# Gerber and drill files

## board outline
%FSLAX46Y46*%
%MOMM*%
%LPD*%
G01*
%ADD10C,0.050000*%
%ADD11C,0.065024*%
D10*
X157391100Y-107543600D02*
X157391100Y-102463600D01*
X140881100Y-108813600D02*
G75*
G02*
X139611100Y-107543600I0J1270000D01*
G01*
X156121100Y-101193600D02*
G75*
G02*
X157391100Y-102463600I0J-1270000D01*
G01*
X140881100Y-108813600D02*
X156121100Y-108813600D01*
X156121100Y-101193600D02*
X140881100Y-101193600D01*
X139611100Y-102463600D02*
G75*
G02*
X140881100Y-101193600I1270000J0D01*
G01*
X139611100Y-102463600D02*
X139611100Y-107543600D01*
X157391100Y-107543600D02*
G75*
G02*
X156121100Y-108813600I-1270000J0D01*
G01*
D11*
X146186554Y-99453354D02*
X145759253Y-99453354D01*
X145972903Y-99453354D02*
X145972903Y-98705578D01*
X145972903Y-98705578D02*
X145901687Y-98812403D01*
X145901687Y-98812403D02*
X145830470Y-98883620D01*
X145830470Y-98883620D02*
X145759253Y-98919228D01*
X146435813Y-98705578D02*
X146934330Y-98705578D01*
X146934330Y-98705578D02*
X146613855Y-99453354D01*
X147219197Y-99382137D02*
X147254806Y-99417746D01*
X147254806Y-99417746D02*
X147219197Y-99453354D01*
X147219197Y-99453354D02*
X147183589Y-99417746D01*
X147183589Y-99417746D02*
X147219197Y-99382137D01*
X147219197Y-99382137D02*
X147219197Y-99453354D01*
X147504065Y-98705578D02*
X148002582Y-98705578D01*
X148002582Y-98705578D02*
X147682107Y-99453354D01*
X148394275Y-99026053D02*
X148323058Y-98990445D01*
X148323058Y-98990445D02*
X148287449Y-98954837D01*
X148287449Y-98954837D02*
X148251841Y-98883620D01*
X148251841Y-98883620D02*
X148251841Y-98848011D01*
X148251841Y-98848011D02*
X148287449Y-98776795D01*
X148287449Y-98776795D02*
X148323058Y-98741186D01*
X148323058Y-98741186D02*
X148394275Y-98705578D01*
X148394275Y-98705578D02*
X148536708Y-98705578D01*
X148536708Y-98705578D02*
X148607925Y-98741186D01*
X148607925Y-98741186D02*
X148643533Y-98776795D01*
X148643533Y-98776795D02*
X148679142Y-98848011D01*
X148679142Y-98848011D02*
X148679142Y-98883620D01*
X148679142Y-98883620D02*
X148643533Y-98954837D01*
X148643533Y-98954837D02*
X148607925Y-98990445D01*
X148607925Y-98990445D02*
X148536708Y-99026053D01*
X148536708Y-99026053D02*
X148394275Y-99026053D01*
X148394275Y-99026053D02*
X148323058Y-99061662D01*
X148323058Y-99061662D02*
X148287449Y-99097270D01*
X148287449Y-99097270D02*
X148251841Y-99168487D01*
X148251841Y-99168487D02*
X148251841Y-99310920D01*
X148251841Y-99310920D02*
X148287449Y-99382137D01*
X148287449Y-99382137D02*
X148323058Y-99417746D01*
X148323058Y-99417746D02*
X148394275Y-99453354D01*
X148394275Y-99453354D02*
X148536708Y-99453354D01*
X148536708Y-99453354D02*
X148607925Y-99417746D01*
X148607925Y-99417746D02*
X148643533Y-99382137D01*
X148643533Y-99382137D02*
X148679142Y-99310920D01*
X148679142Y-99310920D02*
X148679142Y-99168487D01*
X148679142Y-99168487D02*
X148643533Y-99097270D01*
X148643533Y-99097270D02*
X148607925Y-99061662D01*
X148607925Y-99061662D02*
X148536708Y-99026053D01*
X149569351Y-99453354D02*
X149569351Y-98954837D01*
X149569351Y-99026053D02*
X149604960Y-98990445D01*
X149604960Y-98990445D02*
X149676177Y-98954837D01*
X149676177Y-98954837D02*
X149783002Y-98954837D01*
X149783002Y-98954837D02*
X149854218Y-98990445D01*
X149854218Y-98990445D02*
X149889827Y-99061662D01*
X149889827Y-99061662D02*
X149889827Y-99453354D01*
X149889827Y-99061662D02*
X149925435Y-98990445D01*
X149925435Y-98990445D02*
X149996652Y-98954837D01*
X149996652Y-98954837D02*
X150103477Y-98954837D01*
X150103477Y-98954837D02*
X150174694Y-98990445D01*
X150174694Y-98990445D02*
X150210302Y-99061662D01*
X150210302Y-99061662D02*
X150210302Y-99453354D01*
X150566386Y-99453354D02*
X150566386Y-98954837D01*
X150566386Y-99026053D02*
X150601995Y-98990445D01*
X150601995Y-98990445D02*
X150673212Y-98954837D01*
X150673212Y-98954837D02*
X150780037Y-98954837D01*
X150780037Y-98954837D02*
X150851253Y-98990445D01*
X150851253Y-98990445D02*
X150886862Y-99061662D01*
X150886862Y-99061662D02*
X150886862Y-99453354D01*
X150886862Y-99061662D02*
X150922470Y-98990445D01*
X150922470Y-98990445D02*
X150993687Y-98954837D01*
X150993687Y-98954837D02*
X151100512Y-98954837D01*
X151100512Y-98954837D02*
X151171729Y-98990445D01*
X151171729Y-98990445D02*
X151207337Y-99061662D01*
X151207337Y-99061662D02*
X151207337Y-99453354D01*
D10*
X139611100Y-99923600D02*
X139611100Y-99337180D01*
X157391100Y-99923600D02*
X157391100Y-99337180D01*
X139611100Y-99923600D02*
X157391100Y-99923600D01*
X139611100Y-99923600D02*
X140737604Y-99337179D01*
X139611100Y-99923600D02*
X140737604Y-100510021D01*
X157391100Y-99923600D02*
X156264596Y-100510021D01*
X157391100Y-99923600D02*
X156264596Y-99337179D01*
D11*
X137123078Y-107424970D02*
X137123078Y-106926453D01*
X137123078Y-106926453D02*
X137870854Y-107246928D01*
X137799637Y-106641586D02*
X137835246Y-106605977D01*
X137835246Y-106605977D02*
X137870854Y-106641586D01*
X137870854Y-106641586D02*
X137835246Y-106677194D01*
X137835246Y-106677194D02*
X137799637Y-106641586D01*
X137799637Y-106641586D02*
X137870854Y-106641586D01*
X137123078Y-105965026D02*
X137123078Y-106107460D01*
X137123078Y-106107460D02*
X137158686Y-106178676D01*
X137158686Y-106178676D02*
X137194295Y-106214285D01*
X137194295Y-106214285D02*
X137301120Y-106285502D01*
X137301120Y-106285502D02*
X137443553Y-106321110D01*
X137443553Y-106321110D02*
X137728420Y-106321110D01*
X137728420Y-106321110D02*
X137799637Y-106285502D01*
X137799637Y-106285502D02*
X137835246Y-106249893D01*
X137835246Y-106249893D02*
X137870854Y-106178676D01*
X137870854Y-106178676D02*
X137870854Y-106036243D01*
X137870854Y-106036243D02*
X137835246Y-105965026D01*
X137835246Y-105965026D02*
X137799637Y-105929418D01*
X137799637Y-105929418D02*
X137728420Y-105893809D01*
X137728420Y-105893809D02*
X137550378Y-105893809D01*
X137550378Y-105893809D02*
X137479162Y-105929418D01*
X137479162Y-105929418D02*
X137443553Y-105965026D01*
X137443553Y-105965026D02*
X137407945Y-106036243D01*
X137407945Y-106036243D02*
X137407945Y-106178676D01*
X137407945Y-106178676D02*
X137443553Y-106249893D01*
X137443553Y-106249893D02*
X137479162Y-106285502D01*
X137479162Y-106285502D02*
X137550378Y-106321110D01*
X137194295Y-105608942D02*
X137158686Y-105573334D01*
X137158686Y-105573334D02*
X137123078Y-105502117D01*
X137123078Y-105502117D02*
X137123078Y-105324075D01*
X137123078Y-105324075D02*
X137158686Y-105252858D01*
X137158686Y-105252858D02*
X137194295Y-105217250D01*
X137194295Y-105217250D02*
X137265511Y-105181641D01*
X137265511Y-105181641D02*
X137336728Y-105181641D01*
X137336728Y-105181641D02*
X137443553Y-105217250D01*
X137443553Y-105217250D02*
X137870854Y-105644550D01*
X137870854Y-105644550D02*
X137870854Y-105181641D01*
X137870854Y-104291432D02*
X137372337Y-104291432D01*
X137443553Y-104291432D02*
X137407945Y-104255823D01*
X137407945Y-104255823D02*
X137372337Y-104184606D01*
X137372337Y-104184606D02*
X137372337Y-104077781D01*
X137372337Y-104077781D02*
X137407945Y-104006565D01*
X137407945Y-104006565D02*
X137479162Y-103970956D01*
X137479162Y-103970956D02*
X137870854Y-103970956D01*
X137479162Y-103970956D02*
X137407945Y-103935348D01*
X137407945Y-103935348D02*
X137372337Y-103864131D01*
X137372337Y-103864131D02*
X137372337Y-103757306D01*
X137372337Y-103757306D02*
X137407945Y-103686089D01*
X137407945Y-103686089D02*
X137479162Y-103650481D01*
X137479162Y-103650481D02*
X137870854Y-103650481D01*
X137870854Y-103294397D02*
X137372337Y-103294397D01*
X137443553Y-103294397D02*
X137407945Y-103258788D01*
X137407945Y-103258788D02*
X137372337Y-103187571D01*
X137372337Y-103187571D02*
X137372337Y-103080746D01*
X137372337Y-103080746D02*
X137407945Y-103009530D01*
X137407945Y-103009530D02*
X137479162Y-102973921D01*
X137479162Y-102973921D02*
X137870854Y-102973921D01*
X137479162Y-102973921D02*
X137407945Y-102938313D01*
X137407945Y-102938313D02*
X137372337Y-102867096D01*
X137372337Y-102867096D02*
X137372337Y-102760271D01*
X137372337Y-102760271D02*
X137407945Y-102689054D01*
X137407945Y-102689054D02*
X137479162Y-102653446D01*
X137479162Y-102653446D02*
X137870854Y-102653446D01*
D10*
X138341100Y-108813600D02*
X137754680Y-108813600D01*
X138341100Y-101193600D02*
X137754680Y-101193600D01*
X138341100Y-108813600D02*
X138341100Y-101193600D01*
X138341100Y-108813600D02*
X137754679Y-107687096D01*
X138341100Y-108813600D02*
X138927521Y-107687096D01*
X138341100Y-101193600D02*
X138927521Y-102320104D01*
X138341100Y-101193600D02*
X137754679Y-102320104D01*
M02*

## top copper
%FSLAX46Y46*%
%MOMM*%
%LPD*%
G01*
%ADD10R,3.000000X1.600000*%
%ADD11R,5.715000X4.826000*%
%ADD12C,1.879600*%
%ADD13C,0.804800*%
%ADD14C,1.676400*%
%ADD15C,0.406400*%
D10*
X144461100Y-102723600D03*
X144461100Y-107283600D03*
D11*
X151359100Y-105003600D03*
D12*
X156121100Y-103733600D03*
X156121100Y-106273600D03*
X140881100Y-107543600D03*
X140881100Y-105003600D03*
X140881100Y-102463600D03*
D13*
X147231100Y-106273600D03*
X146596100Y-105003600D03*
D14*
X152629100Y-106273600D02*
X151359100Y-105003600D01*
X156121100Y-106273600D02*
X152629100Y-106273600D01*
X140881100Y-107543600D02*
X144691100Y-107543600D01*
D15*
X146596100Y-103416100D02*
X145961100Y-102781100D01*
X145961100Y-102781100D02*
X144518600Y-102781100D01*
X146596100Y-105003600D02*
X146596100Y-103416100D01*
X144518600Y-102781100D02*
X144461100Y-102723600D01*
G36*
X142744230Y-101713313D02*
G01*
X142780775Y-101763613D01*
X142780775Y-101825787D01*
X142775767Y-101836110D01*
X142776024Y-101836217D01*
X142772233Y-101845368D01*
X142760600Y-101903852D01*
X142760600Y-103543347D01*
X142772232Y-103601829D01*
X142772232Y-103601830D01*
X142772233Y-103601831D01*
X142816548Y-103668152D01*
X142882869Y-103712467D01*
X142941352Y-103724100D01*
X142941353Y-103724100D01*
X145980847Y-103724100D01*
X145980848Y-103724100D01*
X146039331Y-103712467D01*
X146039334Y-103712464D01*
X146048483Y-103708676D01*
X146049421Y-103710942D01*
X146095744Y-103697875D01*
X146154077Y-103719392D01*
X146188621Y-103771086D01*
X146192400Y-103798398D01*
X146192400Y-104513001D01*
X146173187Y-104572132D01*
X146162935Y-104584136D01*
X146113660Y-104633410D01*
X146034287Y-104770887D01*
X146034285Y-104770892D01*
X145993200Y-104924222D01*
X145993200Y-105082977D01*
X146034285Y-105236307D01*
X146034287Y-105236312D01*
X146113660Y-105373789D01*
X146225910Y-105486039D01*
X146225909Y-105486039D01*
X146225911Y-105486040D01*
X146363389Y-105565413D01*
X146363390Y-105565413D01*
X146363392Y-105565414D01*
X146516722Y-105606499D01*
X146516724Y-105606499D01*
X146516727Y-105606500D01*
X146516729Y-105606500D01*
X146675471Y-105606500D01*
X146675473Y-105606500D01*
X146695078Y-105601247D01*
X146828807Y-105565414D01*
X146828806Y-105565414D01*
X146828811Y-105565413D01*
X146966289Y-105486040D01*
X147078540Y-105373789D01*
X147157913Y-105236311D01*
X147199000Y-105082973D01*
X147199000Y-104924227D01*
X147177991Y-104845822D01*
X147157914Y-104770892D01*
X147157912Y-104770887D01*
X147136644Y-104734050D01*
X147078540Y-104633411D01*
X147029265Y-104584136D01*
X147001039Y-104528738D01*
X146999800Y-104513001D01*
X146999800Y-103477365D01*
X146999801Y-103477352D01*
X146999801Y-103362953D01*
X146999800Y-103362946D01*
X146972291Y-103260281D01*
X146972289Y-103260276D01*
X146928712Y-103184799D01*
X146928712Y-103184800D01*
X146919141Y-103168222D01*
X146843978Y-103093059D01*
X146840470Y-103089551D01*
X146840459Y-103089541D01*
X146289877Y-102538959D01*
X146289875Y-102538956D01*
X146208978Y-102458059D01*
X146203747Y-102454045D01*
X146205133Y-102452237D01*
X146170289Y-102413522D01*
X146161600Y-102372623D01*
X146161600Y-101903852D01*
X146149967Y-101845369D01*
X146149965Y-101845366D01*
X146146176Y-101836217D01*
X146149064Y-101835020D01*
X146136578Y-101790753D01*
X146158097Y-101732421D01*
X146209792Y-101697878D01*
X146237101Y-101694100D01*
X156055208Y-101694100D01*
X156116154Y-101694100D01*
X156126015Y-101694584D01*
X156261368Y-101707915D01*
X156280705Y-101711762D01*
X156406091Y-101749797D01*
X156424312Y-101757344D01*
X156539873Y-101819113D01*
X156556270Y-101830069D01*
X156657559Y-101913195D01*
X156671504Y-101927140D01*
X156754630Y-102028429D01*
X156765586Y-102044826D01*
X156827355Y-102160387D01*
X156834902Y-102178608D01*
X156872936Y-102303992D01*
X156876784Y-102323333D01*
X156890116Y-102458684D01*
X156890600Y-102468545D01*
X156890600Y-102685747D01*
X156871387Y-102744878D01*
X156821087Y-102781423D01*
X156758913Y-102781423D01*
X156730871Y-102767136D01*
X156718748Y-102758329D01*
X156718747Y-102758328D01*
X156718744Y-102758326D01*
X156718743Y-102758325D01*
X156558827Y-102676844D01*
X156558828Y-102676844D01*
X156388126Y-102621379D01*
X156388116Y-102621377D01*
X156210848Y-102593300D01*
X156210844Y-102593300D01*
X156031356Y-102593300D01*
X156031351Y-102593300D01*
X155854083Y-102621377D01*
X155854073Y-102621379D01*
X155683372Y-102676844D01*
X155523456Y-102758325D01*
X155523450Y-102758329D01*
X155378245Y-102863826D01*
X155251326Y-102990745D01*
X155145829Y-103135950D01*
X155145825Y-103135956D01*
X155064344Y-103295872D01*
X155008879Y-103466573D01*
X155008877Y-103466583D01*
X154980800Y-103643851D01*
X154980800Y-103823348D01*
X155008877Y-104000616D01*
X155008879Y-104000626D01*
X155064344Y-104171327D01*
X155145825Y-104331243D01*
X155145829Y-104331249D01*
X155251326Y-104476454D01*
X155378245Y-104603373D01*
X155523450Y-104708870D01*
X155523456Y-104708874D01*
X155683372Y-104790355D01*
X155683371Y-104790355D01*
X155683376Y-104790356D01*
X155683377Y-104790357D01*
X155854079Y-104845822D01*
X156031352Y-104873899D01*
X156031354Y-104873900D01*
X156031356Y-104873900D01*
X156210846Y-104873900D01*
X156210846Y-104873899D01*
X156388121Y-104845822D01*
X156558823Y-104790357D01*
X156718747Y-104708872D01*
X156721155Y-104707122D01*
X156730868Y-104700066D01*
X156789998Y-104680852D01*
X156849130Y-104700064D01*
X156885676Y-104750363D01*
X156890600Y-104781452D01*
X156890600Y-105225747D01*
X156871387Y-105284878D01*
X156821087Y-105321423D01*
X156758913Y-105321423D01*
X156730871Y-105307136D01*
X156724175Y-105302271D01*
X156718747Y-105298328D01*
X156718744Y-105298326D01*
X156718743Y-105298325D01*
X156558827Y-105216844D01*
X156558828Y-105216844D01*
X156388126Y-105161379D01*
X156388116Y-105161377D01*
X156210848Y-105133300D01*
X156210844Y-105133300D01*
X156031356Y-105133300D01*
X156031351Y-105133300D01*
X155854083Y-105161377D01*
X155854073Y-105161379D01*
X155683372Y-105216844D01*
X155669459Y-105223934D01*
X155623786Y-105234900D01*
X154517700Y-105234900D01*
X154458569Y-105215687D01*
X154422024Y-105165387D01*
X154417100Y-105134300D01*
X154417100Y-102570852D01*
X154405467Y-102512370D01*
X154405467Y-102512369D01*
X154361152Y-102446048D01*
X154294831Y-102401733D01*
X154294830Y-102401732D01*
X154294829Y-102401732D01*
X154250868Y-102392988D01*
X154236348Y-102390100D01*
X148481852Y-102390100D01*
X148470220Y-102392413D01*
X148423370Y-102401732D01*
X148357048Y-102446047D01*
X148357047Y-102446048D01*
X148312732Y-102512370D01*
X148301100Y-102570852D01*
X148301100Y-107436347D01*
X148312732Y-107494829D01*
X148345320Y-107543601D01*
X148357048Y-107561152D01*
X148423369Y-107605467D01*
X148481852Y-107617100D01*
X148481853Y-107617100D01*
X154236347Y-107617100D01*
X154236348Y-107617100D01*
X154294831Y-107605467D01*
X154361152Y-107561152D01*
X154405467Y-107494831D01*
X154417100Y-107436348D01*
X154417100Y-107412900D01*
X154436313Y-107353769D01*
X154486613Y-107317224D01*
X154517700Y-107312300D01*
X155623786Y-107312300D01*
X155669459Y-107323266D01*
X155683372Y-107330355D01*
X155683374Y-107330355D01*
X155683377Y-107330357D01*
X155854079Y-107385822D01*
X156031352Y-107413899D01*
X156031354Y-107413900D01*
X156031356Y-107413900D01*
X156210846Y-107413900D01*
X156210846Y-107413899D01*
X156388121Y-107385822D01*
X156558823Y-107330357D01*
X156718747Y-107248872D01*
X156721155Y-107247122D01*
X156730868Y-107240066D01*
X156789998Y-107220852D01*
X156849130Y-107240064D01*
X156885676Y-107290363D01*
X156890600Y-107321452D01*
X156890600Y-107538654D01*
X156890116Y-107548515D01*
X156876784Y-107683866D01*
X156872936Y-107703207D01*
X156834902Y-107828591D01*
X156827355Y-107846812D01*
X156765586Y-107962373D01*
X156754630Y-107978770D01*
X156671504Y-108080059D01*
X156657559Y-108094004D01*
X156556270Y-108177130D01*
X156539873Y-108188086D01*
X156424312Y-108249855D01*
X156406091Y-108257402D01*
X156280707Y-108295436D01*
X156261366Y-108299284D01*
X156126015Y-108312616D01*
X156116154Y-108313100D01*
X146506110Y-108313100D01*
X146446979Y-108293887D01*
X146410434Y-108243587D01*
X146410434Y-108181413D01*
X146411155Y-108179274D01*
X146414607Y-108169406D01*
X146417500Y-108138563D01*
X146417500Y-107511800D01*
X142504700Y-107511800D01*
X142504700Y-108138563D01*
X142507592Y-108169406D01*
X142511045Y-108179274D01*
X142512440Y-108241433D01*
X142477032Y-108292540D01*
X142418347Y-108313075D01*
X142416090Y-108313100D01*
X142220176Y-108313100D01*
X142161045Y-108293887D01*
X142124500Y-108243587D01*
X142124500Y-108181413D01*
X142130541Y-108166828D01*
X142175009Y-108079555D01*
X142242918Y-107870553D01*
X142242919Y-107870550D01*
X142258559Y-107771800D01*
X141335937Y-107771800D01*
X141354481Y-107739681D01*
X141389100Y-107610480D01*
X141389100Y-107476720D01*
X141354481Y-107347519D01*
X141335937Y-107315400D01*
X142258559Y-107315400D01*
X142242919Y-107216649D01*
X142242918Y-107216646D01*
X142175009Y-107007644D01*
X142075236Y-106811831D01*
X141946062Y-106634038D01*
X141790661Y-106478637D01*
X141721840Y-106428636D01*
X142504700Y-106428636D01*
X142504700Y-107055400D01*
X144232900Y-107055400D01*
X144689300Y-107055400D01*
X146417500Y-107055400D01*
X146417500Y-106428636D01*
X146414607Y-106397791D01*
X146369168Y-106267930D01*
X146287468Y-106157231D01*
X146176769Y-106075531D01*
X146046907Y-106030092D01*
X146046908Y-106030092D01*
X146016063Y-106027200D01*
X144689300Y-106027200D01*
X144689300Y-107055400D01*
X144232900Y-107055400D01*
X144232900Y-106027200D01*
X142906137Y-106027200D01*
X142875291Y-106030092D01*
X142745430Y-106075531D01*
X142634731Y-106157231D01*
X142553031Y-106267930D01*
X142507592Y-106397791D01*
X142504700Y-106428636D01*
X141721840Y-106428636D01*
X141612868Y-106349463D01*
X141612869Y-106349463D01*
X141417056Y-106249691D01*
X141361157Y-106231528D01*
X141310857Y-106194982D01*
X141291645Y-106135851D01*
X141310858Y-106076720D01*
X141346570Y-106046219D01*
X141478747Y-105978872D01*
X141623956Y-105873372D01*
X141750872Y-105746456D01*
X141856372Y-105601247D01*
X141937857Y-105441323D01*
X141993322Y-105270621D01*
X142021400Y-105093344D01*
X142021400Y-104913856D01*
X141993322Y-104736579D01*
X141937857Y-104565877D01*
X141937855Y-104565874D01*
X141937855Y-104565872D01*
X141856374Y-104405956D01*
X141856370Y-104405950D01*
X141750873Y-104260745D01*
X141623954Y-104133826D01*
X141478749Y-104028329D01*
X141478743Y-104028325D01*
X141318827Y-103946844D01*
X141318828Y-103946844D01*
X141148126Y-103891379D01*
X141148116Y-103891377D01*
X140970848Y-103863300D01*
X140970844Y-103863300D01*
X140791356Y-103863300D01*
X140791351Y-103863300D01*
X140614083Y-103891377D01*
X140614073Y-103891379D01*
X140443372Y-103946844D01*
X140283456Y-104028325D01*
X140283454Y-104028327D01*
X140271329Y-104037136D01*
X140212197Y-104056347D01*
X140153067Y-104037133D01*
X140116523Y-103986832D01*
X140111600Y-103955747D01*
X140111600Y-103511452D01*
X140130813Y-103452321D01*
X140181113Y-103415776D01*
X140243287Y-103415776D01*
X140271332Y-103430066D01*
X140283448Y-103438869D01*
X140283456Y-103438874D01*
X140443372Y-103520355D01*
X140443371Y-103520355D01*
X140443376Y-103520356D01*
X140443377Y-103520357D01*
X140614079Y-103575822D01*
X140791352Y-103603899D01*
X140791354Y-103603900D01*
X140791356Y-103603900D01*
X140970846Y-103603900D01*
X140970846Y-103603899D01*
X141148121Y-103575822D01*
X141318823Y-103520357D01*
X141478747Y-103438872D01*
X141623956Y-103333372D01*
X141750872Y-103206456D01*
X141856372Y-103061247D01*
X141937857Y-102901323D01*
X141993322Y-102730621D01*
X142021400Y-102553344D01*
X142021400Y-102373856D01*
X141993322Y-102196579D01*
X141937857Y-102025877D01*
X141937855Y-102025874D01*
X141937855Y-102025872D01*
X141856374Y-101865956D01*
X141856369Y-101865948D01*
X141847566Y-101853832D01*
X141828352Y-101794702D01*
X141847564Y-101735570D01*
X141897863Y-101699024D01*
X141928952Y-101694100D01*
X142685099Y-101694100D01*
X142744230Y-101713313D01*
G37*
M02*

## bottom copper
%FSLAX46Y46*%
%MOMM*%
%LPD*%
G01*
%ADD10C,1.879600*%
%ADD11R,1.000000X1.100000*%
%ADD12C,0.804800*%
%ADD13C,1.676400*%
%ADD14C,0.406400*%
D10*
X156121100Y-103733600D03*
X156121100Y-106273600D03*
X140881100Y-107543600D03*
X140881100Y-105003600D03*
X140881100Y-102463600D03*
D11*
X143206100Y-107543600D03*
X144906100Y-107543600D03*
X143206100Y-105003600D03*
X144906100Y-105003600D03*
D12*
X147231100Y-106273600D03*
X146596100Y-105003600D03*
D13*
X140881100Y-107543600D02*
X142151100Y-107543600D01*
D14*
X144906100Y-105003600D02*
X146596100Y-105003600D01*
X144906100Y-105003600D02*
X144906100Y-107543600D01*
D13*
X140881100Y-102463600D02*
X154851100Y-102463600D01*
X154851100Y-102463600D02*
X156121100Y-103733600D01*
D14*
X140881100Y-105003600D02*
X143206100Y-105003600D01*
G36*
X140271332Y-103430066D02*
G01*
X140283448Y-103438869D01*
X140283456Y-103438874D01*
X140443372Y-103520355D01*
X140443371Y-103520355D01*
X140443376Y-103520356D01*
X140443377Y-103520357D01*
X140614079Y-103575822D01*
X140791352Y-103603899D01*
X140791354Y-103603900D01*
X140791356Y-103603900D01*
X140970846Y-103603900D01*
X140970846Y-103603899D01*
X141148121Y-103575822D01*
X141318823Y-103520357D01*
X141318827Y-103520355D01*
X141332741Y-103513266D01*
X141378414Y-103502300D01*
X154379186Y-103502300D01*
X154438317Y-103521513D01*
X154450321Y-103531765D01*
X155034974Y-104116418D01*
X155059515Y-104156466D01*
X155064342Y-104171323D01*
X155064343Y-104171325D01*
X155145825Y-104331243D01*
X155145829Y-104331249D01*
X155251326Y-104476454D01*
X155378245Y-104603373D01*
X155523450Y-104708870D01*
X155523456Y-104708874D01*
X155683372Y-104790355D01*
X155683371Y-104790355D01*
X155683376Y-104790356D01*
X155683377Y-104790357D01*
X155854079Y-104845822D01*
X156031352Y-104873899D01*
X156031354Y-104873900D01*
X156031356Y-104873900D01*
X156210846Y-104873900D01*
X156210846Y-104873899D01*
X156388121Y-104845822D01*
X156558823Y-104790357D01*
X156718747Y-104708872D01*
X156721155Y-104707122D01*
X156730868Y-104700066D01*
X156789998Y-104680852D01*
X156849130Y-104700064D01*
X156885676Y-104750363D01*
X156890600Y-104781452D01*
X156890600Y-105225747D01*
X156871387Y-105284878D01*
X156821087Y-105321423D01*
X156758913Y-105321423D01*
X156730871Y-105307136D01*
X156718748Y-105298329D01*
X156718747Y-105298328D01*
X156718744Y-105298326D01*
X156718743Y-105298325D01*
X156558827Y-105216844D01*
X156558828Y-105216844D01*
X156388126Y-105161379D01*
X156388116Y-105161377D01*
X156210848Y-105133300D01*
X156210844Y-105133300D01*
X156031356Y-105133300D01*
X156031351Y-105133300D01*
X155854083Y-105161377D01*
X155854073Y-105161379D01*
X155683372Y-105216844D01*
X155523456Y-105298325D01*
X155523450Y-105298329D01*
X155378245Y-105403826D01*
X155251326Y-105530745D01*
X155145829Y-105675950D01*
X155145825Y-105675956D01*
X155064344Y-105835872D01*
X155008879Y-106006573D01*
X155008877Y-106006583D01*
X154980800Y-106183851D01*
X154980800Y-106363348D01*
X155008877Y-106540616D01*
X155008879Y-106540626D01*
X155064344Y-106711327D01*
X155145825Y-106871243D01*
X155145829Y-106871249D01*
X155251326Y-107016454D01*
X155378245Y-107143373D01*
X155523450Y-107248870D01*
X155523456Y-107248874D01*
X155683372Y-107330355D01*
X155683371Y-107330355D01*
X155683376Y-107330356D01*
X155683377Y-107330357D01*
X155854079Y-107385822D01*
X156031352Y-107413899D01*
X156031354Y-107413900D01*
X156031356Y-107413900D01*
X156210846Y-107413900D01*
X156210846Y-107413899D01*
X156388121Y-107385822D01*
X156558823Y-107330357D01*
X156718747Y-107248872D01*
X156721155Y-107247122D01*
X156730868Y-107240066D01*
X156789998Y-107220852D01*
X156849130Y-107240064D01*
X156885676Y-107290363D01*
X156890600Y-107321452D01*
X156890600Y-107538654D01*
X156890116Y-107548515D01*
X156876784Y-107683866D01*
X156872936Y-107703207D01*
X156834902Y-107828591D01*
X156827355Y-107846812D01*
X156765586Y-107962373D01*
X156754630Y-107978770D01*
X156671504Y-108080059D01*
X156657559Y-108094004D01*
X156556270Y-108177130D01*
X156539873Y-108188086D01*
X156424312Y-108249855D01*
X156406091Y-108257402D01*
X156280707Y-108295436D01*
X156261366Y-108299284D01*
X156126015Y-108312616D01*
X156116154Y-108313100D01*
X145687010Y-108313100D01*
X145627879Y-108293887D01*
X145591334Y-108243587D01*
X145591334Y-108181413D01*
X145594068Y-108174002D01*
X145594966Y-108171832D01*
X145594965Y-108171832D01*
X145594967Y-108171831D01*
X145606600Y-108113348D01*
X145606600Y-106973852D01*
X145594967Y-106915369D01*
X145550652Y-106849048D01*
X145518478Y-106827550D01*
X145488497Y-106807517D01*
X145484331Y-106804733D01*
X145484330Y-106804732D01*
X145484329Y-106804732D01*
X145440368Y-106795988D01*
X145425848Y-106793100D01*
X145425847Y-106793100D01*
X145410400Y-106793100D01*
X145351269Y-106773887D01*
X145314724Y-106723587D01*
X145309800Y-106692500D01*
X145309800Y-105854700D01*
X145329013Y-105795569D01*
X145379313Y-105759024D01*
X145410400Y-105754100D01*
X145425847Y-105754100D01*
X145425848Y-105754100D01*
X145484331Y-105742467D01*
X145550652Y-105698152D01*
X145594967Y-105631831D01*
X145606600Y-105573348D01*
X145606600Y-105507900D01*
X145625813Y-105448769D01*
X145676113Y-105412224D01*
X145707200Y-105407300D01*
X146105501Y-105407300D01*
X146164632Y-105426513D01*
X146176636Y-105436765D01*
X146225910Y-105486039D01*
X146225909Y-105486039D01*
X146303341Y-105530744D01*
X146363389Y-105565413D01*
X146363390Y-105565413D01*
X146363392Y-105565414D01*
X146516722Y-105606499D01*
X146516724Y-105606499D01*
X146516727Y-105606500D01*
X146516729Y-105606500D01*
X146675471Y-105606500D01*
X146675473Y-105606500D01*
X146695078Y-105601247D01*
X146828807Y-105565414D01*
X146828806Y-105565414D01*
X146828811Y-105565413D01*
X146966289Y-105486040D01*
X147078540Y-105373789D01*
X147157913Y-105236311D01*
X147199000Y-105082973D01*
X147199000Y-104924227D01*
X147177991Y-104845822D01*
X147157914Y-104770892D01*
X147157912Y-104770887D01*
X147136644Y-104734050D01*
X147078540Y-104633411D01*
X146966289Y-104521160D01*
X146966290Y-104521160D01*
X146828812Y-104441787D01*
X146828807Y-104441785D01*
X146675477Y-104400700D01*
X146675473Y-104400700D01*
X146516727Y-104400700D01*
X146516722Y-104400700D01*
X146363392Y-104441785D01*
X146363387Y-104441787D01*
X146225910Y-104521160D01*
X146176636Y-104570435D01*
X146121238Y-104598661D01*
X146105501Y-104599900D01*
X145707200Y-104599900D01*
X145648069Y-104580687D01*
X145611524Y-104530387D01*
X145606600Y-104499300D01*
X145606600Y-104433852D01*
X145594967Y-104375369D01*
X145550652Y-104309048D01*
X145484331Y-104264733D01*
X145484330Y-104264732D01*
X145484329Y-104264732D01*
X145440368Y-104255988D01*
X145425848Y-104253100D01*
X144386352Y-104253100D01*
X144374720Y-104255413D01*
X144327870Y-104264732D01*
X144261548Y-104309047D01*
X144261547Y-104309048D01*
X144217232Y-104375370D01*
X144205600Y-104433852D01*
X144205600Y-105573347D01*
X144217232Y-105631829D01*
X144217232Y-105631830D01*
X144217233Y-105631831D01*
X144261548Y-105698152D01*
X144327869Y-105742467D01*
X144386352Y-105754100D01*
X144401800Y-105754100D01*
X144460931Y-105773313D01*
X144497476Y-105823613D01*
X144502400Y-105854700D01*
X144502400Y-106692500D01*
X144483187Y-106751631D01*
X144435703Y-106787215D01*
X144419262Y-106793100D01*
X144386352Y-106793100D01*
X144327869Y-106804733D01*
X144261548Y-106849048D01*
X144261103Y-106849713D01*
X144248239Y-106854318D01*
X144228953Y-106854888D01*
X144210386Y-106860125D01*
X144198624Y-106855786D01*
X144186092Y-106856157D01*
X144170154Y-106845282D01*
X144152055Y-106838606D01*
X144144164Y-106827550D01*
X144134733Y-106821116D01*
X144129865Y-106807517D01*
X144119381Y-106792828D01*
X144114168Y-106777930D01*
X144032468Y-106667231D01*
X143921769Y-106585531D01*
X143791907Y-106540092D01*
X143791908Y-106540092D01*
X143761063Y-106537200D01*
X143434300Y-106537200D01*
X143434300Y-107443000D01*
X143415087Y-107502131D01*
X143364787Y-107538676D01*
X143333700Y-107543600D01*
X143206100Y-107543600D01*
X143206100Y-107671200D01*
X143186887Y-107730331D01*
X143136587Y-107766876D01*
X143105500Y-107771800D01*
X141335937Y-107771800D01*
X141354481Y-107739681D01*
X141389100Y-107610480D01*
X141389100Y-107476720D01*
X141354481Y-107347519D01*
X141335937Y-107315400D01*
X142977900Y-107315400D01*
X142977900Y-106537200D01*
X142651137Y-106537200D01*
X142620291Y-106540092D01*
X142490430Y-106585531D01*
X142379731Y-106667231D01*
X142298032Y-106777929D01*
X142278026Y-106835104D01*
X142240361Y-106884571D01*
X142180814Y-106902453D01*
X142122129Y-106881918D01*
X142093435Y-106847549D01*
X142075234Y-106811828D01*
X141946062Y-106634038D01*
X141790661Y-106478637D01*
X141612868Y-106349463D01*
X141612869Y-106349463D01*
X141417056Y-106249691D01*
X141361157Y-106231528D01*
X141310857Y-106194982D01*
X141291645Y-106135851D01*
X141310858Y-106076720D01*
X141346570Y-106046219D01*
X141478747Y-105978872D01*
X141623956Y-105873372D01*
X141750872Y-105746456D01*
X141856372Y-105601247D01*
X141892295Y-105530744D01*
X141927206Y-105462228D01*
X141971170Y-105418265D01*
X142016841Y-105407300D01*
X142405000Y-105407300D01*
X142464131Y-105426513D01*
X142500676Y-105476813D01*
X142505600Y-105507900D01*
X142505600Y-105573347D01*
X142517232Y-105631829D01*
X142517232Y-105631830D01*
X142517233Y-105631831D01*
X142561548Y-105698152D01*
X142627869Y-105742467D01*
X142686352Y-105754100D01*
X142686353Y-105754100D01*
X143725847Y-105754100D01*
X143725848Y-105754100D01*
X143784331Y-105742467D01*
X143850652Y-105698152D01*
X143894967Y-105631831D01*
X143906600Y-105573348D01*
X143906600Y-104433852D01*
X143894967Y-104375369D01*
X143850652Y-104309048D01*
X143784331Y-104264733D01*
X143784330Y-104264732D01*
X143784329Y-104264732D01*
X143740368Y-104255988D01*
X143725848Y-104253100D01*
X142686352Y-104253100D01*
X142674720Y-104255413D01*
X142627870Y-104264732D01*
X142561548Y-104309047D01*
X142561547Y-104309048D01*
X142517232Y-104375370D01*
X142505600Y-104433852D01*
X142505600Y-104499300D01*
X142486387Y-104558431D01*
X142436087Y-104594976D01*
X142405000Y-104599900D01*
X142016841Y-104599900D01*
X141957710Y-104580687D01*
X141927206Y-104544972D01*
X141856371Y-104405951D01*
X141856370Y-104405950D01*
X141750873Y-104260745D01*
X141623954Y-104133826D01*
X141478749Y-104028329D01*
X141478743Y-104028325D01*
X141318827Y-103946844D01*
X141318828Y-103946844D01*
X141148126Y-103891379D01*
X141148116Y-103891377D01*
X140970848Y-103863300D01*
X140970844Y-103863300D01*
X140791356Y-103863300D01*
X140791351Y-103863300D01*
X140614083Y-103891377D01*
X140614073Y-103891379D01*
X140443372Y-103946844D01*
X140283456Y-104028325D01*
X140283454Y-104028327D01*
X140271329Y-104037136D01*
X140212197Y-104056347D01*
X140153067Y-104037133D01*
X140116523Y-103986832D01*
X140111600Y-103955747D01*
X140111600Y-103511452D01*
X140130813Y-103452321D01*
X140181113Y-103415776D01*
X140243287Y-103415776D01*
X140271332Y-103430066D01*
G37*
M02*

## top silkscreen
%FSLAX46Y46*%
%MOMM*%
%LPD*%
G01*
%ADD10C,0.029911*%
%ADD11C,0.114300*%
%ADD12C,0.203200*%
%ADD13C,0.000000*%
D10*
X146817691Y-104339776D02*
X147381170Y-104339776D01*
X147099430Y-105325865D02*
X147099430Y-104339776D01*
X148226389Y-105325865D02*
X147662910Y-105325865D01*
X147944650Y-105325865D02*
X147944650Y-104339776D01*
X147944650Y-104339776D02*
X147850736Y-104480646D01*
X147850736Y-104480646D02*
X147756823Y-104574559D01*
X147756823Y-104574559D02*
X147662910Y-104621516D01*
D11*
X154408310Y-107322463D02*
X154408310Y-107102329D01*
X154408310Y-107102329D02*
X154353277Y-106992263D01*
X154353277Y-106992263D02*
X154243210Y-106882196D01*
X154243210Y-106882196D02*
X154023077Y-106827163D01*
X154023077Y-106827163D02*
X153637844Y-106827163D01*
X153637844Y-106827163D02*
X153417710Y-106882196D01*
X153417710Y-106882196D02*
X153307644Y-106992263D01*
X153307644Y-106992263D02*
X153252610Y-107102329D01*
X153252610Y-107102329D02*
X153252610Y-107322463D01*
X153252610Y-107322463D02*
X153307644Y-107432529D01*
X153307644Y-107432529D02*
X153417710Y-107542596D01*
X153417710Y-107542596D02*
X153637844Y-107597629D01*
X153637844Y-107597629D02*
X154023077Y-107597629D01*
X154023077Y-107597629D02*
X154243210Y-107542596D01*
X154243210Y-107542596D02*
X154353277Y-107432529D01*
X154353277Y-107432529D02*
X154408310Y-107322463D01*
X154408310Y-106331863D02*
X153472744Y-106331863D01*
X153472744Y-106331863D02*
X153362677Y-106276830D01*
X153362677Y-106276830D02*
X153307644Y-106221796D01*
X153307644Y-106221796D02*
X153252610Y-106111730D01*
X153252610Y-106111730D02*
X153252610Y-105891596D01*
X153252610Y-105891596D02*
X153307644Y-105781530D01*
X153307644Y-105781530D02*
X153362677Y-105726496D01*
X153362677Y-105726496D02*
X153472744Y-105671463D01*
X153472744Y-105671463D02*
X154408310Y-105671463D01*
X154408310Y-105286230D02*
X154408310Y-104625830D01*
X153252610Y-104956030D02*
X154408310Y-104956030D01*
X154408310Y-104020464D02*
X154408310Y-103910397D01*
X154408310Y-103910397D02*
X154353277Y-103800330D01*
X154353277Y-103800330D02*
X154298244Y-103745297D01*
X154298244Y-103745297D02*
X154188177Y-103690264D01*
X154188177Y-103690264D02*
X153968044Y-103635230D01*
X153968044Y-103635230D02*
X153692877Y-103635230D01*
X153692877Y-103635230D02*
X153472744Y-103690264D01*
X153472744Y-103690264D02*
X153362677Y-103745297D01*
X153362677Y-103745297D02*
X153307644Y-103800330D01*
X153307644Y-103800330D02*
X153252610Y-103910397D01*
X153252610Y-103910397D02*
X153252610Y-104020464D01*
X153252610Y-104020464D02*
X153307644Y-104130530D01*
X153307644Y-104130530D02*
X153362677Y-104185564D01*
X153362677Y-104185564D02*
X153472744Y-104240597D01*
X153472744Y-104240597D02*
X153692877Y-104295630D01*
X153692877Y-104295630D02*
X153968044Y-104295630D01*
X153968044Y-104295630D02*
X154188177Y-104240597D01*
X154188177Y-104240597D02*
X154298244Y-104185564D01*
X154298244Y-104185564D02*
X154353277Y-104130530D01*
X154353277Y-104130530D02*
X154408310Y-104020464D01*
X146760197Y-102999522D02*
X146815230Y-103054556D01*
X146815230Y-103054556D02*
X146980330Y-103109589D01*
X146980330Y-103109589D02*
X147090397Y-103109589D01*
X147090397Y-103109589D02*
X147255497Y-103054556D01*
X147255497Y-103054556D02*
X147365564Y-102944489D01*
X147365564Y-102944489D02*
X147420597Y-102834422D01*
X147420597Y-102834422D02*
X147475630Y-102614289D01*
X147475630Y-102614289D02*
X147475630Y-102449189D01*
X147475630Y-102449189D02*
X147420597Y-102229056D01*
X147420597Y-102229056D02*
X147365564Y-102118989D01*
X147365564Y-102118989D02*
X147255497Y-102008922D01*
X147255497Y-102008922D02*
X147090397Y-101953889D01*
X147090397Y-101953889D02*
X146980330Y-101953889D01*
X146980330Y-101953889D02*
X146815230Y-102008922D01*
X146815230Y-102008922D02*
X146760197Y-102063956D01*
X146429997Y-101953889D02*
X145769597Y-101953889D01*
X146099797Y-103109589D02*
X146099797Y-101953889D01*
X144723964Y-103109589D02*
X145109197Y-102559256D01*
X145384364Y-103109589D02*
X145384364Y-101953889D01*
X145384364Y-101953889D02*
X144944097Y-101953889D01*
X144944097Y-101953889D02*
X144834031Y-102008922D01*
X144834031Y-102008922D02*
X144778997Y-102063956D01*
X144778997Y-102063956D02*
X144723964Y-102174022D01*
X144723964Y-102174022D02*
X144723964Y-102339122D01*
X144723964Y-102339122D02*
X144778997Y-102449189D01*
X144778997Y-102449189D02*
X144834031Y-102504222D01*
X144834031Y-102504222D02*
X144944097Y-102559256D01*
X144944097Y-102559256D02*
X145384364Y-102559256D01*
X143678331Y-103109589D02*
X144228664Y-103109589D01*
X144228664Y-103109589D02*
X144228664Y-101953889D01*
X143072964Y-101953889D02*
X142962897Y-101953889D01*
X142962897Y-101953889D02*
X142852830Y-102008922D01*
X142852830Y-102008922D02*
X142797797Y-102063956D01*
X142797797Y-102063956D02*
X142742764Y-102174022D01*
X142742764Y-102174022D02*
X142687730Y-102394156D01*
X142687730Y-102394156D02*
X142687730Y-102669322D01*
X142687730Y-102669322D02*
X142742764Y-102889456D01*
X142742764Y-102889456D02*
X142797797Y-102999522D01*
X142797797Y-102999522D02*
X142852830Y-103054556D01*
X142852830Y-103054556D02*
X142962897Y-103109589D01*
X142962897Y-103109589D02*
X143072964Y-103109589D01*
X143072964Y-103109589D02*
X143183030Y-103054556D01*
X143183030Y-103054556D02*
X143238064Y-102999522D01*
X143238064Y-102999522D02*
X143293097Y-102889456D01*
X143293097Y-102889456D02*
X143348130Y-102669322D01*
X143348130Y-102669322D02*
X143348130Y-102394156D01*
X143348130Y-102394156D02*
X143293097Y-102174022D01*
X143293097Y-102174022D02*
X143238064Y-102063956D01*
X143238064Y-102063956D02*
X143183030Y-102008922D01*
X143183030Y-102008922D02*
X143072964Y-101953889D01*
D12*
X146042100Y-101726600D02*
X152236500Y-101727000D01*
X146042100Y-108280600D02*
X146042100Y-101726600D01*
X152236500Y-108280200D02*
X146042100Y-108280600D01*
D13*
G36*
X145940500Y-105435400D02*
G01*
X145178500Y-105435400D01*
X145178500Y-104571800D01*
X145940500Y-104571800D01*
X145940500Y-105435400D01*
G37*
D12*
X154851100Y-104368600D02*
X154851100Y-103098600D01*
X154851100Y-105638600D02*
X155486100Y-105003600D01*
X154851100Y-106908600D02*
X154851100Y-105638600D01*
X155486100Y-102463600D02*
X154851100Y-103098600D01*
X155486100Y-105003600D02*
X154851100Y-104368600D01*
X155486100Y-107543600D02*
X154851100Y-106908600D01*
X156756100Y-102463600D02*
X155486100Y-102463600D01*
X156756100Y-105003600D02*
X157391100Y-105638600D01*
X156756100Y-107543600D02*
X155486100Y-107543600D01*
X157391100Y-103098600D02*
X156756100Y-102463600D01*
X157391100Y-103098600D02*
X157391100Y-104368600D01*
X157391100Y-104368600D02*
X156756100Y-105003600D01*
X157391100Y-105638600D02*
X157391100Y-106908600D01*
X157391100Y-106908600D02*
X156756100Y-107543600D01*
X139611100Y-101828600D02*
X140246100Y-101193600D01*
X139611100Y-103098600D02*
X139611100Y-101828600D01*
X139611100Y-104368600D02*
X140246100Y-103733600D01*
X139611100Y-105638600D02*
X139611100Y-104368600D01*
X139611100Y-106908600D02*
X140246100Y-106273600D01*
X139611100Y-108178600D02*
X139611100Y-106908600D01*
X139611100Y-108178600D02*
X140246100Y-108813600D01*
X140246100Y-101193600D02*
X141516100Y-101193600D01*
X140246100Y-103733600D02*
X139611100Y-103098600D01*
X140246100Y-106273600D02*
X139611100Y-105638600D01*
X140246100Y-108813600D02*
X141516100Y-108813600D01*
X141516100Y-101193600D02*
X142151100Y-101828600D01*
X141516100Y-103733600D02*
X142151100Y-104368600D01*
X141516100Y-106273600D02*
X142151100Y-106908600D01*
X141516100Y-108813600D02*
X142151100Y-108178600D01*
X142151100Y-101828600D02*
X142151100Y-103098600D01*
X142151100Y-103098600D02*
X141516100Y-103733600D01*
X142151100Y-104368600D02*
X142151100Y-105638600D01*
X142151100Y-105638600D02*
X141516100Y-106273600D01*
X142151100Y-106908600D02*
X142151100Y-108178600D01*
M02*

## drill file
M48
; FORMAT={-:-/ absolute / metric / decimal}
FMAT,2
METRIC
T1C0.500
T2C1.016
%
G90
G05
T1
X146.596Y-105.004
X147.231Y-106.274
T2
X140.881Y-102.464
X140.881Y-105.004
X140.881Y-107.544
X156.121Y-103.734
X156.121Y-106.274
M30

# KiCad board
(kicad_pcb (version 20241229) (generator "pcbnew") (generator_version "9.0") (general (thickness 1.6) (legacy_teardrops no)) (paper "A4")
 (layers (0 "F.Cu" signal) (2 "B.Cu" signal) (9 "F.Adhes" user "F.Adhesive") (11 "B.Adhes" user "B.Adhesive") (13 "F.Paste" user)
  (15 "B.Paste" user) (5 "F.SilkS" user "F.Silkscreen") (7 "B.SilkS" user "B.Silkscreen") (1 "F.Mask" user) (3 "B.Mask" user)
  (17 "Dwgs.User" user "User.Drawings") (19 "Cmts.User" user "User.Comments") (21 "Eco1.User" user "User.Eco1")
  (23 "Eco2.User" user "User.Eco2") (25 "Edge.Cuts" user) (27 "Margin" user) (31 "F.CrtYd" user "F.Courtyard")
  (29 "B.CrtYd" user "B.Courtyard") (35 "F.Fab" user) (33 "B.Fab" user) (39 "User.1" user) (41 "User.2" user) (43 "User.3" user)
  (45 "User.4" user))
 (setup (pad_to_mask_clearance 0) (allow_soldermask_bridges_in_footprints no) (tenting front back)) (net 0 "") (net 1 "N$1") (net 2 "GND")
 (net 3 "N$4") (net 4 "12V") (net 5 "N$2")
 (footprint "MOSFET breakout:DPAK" (layer "F.Cu") (at 149.7711 105.0036 -90)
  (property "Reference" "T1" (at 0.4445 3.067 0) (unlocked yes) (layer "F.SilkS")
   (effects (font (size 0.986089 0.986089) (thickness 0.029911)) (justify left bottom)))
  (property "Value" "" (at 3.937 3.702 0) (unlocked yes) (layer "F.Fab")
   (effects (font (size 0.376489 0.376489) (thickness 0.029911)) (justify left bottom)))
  (fp_line (start -3.277 3.729) (end -3.2766 -2.4654) (stroke (width 0.2032) (type solid)) (layer "F.SilkS"))
  (fp_line (start 3.277 3.729) (end -3.277 3.729) (stroke (width 0.2032) (type solid)) (layer "F.SilkS"))
  (fp_line (start 3.2766 -2.4654) (end 3.277 3.729) (stroke (width 0.2032) (type solid)) (layer "F.SilkS"))
  (fp_poly
   (pts (xy -0.4318 4.5926) (xy 0.4318 4.5926) (xy 0.4318 3.8306) (xy -0.4318 3.8306)) (stroke (width 0) (type default)) (fill yes)
   (layer "F.SilkS"))
  (pad "1" smd rect (at -2.28 5.31 270) (size 1.6 3) (layers "F.Cu" "F.Mask" "F.Paste") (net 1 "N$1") (solder_mask_margin 0.0508)
   (solder_paste_margin 0) (thermal_bridge_angle 0))
  (pad "3" smd rect (at 2.28 5.31 270) (size 1.6 3) (layers "F.Cu" "F.Mask" "F.Paste") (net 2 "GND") (solder_mask_margin 0.0508)
   (solder_paste_margin 0) (thermal_bridge_angle 0))
  (pad "4" smd rect (at 0 -1.588 270) (size 4.826 5.715) (layers "F.Cu" "F.Mask" "F.Paste") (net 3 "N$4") (solder_mask_margin 0.0508)
   (solder_paste_margin 0) (thermal_bridge_angle 0)))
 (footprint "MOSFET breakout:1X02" (layer "F.Cu") (at 156.1211 103.7336 -90)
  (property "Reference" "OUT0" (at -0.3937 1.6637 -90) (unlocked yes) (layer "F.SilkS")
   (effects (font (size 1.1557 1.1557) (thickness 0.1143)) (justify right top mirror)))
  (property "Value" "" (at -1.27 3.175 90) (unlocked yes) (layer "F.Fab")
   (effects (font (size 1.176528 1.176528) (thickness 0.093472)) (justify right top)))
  (fp_line (start 0.635 1.27) (end -0.635 1.27) (stroke (width 0.2032) (type solid)) (layer "F.SilkS"))
  (fp_line (start 1.905 1.27) (end 1.27 0.635) (stroke (width 0.2032) (type solid)) (layer "F.SilkS"))
  (fp_line (start 3.175 1.27) (end 1.905 1.27) (stroke (width 0.2032) (type solid)) (layer "F.SilkS"))
  (fp_line (start -1.27 0.635) (end -0.635 1.27) (stroke (width 0.2032) (type solid)) (layer "F.SilkS"))
  (fp_line (start 1.27 0.635) (end 0.635 1.27) (stroke (width 0.2032) (type solid)) (layer "F.SilkS"))
  (fp_line (start 3.81 0.635) (end 3.175 1.27) (stroke (width 0.2032) (type solid)) (layer "F.SilkS"))
  (fp_line (start -1.27 -0.635) (end -1.27 0.635) (stroke (width 0.2032) (type solid)) (layer "F.SilkS"))
  (fp_line (start 1.27 -0.635) (end 1.905 -1.27) (stroke (width 0.2032) (type solid)) (layer "F.SilkS"))
  (fp_line (start 3.81 -0.635) (end 3.81 0.635) (stroke (width 0.2032) (type solid)) (layer "F.SilkS"))
  (fp_line (start -0.635 -1.27) (end -1.27 -0.635) (stroke (width 0.2032) (type solid)) (layer "F.SilkS"))
  (fp_line (start -0.635 -1.27) (end 0.635 -1.27) (stroke (width 0.2032) (type solid)) (layer "F.SilkS"))
  (fp_line (start 0.635 -1.27) (end 1.27 -0.635) (stroke (width 0.2032) (type solid)) (layer "F.SilkS"))
  (fp_line (start 1.905 -1.27) (end 3.175 -1.27) (stroke (width 0.2032) (type solid)) (layer "F.SilkS"))
  (fp_line (start 3.175 -1.27) (end 3.81 -0.635) (stroke (width 0.2032) (type solid)) (layer "F.SilkS"))
  (pad "1" thru_hole circle (at 0 0) (size 1.8796 1.8796) (drill 1.016) (layers "*.Cu" "*.Mask") (remove_unused_layers no) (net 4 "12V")
   (solder_mask_margin 0.0508) (thermal_bridge_angle 0))
  (pad "2" thru_hole circle (at 2.54 0) (size 1.8796 1.8796) (drill 1.016) (layers "*.Cu" "*.Mask") (remove_unused_layers no) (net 3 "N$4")
   (solder_mask_margin 0.0508) (thermal_bridge_angle 0)))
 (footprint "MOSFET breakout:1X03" (layer "F.Cu") (at 140.8811 107.5436 90)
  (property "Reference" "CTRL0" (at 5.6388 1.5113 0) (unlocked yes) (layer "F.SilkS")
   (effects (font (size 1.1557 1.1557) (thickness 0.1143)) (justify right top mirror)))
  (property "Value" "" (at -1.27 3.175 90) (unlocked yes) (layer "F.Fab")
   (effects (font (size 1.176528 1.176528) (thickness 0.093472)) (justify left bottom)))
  (fp_line (start 5.715 -1.27) (end 6.35 -0.635) (stroke (width 0.2032) (type solid)) (layer "F.SilkS"))
  (fp_line (start 4.445 -1.27) (end 5.715 -1.27) (stroke (width 0.2032) (type solid)) (layer "F.SilkS"))
  (fp_line (start 3.175 -1.27) (end 3.81 -0.635) (stroke (width 0.2032) (type solid)) (layer "F.SilkS"))
  (fp_line (start 1.905 -1.27) (end 3.175 -1.27) (stroke (width 0.2032) (type solid)) (layer "F.SilkS"))
  (fp_line (start 0.635 -1.27) (end 1.27 -0.635) (stroke (width 0.2032) (type solid)) (layer "F.SilkS"))
  (fp_line (start -0.635 -1.27) (end 0.635 -1.27) (stroke (width 0.2032) (type solid)) (layer "F.SilkS"))
  (fp_line (start -0.635 -1.27) (end -1.27 -0.635) (stroke (width 0.2032) (type solid)) (layer "F.SilkS"))
  (fp_line (start 6.35 -0.635) (end 6.35 0.635) (stroke (width 0.2032) (type solid)) (layer "F.SilkS"))
  (fp_line (start 3.81 -0.635) (end 4.445 -1.27) (stroke (width 0.2032) (type solid)) (layer "F.SilkS"))
  (fp_line (start 1.27 -0.635) (end 1.905 -1.27) (stroke (width 0.2032) (type solid)) (layer "F.SilkS"))
  (fp_line (start -1.27 -0.635) (end -1.27 0.635) (stroke (width 0.2032) (type solid)) (layer "F.SilkS"))
  (fp_line (start 6.35 0.635) (end 5.715 1.27) (stroke (width 0.2032) (type solid)) (layer "F.SilkS"))
  (fp_line (start 3.81 0.635) (end 3.175 1.27) (stroke (width 0.2032) (type solid)) (layer "F.SilkS"))
  (fp_line (start 1.27 0.635) (end 0.635 1.27) (stroke (width 0.2032) (type solid)) (layer "F.SilkS"))
  (fp_line (start -1.27 0.635) (end -0.635 1.27) (stroke (width 0.2032) (type solid)) (layer "F.SilkS"))
  (fp_line (start 5.715 1.27) (end 4.445 1.27) (stroke (width 0.2032) (type solid)) (layer "F.SilkS"))
  (fp_line (start 4.445 1.27) (end 3.81 0.635) (stroke (width 0.2032) (type solid)) (layer "F.SilkS"))
  (fp_line (start 3.175 1.27) (end 1.905 1.27) (stroke (width 0.2032) (type solid)) (layer "F.SilkS"))
  (fp_line (start 1.905 1.27) (end 1.27 0.635) (stroke (width 0.2032) (type solid)) (layer "F.SilkS"))
  (fp_line (start 0.635 1.27) (end -0.635 1.27) (stroke (width 0.2032) (type solid)) (layer "F.SilkS"))
  (pad "1" thru_hole circle (at 0 0 180) (size 1.8796 1.8796) (drill 1.016) (layers "*.Cu" "*.Mask") (remove_unused_layers no) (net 2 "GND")
   (solder_mask_margin 0.0508) (thermal_bridge_angle 0))
  (pad "2" thru_hole circle (at 2.54 0 180) (size 1.8796 1.8796) (drill 1.016) (layers "*.Cu" "*.Mask") (remove_unused_layers no)
   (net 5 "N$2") (solder_mask_margin 0.0508) (thermal_bridge_angle 0))
  (pad "3" thru_hole circle (at 5.08 0 180) (size 1.8796 1.8796) (drill 1.016) (layers "*.Cu" "*.Mask") (remove_unused_layers no)
   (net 4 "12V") (solder_mask_margin 0.0508) (thermal_bridge_angle 0)))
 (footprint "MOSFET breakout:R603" (layer "B.Cu") (at 144.0561 107.5436)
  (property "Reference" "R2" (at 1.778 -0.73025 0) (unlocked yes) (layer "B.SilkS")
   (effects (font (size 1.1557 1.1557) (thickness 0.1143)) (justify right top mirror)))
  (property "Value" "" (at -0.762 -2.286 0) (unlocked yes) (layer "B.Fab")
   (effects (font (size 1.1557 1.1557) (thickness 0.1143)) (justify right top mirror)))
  (pad "1" smd rect (at -0.85 0) (size 1 1.1) (layers "B.Cu" "B.Mask" "B.Paste") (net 2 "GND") (solder_mask_margin 0.0508)
   (solder_paste_margin 0) (thermal_bridge_angle 0))
  (pad "2" smd rect (at 0.85 0) (size 1 1.1) (layers "B.Cu" "B.Mask" "B.Paste") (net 1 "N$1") (solder_mask_margin 0.0508)
   (solder_paste_margin 0) (thermal_bridge_angle 0)))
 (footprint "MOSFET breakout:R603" (layer "B.Cu") (at 144.0561 105.0036)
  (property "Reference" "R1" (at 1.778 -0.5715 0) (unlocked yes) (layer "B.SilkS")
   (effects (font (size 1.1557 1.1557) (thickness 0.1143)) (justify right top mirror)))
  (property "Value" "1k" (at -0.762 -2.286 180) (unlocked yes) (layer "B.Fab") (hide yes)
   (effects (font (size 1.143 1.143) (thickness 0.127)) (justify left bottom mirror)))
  (pad "1" smd rect (at -0.85 0) (size 1 1.1) (layers "B.Cu" "B.Mask" "B.Paste") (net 5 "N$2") (solder_mask_margin 0.0508)
   (solder_paste_margin 0) (thermal_bridge_angle 0))
  (pad "2" smd rect (at 0.85 0) (size 1 1.1) (layers "B.Cu" "B.Mask" "B.Paste") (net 1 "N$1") (solder_mask_margin 0.0508)
   (solder_paste_margin 0) (thermal_bridge_angle 0)))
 (gr_line (start 157.3911 107.5436) (end 157.3911 102.4636) (stroke (width 0.05) (type solid)) (layer "Edge.Cuts"))
 (gr_arc (start 140.8811 108.8136) (mid 139.983074 108.441626) (end 139.6111 107.5436) (stroke (width 0.05) (type solid))
  (layer "Edge.Cuts"))
 (gr_arc (start 156.1211 101.1936) (mid 157.019126 101.565574) (end 157.3911 102.4636) (stroke (width 0.05) (type solid))
  (layer "Edge.Cuts"))
 (gr_line (start 140.8811 108.8136) (end 156.1211 108.8136) (stroke (width 0.05) (type solid)) (layer "Edge.Cuts"))
 (gr_line (start 156.1211 101.1936) (end 140.8811 101.1936) (stroke (width 0.05) (type solid)) (layer "Edge.Cuts"))
 (gr_arc (start 139.6111 102.4636) (mid 139.983074 101.565574) (end 140.8811 101.1936) (stroke (width 0.05) (type solid))
  (layer "Edge.Cuts"))
 (gr_line (start 139.6111 102.4636) (end 139.6111 107.5436) (stroke (width 0.05) (type solid)) (layer "Edge.Cuts"))
 (gr_arc (start 157.3911 107.5436) (mid 157.019126 108.441626) (end 156.1211 108.8136) (stroke (width 0.05) (type solid))
  (layer "Edge.Cuts"))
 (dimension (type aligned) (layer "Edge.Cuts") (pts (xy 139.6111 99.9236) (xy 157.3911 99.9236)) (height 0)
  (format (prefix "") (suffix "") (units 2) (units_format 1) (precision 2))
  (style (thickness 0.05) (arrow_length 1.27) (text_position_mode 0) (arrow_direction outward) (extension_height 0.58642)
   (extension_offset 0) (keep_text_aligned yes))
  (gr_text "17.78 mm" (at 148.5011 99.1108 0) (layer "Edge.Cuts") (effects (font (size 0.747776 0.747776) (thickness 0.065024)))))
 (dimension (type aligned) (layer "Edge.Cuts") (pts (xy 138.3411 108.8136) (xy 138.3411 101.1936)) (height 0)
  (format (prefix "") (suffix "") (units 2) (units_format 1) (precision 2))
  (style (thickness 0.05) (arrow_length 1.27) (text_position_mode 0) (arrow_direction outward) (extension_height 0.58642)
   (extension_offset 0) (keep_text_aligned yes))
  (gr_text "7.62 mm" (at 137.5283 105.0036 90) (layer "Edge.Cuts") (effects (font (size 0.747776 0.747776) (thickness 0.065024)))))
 (segment (start 152.6291 106.2736) (end 151.3591 105.0036) (width 1.6764) (layer "F.Cu") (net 3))
 (segment (start 156.1211 106.2736) (end 152.6291 106.2736) (width 1.6764) (layer "F.Cu") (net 3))
 (segment (start 140.8811 107.5436) (end 144.6911 107.5436) (width 1.6764) (layer "F.Cu") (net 2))
 (via (at 147.2311 106.2736) (size 0.8048) (drill 0.5) (layers "F.Cu" "B.Cu") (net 2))
 (segment (start 140.8811 107.5436) (end 142.1511 107.5436) (width 1.6764) (layer "B.Cu") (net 2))
 (segment (start 146.5961 103.4161) (end 145.9611 102.7811) (width 0.4064) (layer "F.Cu") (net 1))
 (segment (start 145.9611 102.7811) (end 144.5186 102.7811) (width 0.4064) (layer "F.Cu") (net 1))
 (segment (start 146.5961 105.0036) (end 146.5961 103.4161) (width 0.4064) (layer "F.Cu") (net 1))
 (segment (start 144.5186 102.7811) (end 144.4611 102.7236) (width 0.4064) (layer "F.Cu") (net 1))
 (via (at 146.5961 105.0036) (size 0.8048) (drill 0.5) (layers "F.Cu" "B.Cu") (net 1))
 (segment (start 144.9061 105.0036) (end 146.5961 105.0036) (width 0.4064) (layer "B.Cu") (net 1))
 (segment (start 144.9061 105.0036) (end 144.9061 107.5436) (width 0.4064) (layer "B.Cu") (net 1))
 (segment (start 140.8811 102.4636) (end 154.8511 102.4636) (width 1.6764) (layer "B.Cu") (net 4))
 (segment (start 154.8511 102.4636) (end 156.1211 103.7336) (width 1.6764) (layer "B.Cu") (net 4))
 (segment (start 140.8811 105.0036) (end 143.2061 105.0036) (width 0.4064) (layer "B.Cu") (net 5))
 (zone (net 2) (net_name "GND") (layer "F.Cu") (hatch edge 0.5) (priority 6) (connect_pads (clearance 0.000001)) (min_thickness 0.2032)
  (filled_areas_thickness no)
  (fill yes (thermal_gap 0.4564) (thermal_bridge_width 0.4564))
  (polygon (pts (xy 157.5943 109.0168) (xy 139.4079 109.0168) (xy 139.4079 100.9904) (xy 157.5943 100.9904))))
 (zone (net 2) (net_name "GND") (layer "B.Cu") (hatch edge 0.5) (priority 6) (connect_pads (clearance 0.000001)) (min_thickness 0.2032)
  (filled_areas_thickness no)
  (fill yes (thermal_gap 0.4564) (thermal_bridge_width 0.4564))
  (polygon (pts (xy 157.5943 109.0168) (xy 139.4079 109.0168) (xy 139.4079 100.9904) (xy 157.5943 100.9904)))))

